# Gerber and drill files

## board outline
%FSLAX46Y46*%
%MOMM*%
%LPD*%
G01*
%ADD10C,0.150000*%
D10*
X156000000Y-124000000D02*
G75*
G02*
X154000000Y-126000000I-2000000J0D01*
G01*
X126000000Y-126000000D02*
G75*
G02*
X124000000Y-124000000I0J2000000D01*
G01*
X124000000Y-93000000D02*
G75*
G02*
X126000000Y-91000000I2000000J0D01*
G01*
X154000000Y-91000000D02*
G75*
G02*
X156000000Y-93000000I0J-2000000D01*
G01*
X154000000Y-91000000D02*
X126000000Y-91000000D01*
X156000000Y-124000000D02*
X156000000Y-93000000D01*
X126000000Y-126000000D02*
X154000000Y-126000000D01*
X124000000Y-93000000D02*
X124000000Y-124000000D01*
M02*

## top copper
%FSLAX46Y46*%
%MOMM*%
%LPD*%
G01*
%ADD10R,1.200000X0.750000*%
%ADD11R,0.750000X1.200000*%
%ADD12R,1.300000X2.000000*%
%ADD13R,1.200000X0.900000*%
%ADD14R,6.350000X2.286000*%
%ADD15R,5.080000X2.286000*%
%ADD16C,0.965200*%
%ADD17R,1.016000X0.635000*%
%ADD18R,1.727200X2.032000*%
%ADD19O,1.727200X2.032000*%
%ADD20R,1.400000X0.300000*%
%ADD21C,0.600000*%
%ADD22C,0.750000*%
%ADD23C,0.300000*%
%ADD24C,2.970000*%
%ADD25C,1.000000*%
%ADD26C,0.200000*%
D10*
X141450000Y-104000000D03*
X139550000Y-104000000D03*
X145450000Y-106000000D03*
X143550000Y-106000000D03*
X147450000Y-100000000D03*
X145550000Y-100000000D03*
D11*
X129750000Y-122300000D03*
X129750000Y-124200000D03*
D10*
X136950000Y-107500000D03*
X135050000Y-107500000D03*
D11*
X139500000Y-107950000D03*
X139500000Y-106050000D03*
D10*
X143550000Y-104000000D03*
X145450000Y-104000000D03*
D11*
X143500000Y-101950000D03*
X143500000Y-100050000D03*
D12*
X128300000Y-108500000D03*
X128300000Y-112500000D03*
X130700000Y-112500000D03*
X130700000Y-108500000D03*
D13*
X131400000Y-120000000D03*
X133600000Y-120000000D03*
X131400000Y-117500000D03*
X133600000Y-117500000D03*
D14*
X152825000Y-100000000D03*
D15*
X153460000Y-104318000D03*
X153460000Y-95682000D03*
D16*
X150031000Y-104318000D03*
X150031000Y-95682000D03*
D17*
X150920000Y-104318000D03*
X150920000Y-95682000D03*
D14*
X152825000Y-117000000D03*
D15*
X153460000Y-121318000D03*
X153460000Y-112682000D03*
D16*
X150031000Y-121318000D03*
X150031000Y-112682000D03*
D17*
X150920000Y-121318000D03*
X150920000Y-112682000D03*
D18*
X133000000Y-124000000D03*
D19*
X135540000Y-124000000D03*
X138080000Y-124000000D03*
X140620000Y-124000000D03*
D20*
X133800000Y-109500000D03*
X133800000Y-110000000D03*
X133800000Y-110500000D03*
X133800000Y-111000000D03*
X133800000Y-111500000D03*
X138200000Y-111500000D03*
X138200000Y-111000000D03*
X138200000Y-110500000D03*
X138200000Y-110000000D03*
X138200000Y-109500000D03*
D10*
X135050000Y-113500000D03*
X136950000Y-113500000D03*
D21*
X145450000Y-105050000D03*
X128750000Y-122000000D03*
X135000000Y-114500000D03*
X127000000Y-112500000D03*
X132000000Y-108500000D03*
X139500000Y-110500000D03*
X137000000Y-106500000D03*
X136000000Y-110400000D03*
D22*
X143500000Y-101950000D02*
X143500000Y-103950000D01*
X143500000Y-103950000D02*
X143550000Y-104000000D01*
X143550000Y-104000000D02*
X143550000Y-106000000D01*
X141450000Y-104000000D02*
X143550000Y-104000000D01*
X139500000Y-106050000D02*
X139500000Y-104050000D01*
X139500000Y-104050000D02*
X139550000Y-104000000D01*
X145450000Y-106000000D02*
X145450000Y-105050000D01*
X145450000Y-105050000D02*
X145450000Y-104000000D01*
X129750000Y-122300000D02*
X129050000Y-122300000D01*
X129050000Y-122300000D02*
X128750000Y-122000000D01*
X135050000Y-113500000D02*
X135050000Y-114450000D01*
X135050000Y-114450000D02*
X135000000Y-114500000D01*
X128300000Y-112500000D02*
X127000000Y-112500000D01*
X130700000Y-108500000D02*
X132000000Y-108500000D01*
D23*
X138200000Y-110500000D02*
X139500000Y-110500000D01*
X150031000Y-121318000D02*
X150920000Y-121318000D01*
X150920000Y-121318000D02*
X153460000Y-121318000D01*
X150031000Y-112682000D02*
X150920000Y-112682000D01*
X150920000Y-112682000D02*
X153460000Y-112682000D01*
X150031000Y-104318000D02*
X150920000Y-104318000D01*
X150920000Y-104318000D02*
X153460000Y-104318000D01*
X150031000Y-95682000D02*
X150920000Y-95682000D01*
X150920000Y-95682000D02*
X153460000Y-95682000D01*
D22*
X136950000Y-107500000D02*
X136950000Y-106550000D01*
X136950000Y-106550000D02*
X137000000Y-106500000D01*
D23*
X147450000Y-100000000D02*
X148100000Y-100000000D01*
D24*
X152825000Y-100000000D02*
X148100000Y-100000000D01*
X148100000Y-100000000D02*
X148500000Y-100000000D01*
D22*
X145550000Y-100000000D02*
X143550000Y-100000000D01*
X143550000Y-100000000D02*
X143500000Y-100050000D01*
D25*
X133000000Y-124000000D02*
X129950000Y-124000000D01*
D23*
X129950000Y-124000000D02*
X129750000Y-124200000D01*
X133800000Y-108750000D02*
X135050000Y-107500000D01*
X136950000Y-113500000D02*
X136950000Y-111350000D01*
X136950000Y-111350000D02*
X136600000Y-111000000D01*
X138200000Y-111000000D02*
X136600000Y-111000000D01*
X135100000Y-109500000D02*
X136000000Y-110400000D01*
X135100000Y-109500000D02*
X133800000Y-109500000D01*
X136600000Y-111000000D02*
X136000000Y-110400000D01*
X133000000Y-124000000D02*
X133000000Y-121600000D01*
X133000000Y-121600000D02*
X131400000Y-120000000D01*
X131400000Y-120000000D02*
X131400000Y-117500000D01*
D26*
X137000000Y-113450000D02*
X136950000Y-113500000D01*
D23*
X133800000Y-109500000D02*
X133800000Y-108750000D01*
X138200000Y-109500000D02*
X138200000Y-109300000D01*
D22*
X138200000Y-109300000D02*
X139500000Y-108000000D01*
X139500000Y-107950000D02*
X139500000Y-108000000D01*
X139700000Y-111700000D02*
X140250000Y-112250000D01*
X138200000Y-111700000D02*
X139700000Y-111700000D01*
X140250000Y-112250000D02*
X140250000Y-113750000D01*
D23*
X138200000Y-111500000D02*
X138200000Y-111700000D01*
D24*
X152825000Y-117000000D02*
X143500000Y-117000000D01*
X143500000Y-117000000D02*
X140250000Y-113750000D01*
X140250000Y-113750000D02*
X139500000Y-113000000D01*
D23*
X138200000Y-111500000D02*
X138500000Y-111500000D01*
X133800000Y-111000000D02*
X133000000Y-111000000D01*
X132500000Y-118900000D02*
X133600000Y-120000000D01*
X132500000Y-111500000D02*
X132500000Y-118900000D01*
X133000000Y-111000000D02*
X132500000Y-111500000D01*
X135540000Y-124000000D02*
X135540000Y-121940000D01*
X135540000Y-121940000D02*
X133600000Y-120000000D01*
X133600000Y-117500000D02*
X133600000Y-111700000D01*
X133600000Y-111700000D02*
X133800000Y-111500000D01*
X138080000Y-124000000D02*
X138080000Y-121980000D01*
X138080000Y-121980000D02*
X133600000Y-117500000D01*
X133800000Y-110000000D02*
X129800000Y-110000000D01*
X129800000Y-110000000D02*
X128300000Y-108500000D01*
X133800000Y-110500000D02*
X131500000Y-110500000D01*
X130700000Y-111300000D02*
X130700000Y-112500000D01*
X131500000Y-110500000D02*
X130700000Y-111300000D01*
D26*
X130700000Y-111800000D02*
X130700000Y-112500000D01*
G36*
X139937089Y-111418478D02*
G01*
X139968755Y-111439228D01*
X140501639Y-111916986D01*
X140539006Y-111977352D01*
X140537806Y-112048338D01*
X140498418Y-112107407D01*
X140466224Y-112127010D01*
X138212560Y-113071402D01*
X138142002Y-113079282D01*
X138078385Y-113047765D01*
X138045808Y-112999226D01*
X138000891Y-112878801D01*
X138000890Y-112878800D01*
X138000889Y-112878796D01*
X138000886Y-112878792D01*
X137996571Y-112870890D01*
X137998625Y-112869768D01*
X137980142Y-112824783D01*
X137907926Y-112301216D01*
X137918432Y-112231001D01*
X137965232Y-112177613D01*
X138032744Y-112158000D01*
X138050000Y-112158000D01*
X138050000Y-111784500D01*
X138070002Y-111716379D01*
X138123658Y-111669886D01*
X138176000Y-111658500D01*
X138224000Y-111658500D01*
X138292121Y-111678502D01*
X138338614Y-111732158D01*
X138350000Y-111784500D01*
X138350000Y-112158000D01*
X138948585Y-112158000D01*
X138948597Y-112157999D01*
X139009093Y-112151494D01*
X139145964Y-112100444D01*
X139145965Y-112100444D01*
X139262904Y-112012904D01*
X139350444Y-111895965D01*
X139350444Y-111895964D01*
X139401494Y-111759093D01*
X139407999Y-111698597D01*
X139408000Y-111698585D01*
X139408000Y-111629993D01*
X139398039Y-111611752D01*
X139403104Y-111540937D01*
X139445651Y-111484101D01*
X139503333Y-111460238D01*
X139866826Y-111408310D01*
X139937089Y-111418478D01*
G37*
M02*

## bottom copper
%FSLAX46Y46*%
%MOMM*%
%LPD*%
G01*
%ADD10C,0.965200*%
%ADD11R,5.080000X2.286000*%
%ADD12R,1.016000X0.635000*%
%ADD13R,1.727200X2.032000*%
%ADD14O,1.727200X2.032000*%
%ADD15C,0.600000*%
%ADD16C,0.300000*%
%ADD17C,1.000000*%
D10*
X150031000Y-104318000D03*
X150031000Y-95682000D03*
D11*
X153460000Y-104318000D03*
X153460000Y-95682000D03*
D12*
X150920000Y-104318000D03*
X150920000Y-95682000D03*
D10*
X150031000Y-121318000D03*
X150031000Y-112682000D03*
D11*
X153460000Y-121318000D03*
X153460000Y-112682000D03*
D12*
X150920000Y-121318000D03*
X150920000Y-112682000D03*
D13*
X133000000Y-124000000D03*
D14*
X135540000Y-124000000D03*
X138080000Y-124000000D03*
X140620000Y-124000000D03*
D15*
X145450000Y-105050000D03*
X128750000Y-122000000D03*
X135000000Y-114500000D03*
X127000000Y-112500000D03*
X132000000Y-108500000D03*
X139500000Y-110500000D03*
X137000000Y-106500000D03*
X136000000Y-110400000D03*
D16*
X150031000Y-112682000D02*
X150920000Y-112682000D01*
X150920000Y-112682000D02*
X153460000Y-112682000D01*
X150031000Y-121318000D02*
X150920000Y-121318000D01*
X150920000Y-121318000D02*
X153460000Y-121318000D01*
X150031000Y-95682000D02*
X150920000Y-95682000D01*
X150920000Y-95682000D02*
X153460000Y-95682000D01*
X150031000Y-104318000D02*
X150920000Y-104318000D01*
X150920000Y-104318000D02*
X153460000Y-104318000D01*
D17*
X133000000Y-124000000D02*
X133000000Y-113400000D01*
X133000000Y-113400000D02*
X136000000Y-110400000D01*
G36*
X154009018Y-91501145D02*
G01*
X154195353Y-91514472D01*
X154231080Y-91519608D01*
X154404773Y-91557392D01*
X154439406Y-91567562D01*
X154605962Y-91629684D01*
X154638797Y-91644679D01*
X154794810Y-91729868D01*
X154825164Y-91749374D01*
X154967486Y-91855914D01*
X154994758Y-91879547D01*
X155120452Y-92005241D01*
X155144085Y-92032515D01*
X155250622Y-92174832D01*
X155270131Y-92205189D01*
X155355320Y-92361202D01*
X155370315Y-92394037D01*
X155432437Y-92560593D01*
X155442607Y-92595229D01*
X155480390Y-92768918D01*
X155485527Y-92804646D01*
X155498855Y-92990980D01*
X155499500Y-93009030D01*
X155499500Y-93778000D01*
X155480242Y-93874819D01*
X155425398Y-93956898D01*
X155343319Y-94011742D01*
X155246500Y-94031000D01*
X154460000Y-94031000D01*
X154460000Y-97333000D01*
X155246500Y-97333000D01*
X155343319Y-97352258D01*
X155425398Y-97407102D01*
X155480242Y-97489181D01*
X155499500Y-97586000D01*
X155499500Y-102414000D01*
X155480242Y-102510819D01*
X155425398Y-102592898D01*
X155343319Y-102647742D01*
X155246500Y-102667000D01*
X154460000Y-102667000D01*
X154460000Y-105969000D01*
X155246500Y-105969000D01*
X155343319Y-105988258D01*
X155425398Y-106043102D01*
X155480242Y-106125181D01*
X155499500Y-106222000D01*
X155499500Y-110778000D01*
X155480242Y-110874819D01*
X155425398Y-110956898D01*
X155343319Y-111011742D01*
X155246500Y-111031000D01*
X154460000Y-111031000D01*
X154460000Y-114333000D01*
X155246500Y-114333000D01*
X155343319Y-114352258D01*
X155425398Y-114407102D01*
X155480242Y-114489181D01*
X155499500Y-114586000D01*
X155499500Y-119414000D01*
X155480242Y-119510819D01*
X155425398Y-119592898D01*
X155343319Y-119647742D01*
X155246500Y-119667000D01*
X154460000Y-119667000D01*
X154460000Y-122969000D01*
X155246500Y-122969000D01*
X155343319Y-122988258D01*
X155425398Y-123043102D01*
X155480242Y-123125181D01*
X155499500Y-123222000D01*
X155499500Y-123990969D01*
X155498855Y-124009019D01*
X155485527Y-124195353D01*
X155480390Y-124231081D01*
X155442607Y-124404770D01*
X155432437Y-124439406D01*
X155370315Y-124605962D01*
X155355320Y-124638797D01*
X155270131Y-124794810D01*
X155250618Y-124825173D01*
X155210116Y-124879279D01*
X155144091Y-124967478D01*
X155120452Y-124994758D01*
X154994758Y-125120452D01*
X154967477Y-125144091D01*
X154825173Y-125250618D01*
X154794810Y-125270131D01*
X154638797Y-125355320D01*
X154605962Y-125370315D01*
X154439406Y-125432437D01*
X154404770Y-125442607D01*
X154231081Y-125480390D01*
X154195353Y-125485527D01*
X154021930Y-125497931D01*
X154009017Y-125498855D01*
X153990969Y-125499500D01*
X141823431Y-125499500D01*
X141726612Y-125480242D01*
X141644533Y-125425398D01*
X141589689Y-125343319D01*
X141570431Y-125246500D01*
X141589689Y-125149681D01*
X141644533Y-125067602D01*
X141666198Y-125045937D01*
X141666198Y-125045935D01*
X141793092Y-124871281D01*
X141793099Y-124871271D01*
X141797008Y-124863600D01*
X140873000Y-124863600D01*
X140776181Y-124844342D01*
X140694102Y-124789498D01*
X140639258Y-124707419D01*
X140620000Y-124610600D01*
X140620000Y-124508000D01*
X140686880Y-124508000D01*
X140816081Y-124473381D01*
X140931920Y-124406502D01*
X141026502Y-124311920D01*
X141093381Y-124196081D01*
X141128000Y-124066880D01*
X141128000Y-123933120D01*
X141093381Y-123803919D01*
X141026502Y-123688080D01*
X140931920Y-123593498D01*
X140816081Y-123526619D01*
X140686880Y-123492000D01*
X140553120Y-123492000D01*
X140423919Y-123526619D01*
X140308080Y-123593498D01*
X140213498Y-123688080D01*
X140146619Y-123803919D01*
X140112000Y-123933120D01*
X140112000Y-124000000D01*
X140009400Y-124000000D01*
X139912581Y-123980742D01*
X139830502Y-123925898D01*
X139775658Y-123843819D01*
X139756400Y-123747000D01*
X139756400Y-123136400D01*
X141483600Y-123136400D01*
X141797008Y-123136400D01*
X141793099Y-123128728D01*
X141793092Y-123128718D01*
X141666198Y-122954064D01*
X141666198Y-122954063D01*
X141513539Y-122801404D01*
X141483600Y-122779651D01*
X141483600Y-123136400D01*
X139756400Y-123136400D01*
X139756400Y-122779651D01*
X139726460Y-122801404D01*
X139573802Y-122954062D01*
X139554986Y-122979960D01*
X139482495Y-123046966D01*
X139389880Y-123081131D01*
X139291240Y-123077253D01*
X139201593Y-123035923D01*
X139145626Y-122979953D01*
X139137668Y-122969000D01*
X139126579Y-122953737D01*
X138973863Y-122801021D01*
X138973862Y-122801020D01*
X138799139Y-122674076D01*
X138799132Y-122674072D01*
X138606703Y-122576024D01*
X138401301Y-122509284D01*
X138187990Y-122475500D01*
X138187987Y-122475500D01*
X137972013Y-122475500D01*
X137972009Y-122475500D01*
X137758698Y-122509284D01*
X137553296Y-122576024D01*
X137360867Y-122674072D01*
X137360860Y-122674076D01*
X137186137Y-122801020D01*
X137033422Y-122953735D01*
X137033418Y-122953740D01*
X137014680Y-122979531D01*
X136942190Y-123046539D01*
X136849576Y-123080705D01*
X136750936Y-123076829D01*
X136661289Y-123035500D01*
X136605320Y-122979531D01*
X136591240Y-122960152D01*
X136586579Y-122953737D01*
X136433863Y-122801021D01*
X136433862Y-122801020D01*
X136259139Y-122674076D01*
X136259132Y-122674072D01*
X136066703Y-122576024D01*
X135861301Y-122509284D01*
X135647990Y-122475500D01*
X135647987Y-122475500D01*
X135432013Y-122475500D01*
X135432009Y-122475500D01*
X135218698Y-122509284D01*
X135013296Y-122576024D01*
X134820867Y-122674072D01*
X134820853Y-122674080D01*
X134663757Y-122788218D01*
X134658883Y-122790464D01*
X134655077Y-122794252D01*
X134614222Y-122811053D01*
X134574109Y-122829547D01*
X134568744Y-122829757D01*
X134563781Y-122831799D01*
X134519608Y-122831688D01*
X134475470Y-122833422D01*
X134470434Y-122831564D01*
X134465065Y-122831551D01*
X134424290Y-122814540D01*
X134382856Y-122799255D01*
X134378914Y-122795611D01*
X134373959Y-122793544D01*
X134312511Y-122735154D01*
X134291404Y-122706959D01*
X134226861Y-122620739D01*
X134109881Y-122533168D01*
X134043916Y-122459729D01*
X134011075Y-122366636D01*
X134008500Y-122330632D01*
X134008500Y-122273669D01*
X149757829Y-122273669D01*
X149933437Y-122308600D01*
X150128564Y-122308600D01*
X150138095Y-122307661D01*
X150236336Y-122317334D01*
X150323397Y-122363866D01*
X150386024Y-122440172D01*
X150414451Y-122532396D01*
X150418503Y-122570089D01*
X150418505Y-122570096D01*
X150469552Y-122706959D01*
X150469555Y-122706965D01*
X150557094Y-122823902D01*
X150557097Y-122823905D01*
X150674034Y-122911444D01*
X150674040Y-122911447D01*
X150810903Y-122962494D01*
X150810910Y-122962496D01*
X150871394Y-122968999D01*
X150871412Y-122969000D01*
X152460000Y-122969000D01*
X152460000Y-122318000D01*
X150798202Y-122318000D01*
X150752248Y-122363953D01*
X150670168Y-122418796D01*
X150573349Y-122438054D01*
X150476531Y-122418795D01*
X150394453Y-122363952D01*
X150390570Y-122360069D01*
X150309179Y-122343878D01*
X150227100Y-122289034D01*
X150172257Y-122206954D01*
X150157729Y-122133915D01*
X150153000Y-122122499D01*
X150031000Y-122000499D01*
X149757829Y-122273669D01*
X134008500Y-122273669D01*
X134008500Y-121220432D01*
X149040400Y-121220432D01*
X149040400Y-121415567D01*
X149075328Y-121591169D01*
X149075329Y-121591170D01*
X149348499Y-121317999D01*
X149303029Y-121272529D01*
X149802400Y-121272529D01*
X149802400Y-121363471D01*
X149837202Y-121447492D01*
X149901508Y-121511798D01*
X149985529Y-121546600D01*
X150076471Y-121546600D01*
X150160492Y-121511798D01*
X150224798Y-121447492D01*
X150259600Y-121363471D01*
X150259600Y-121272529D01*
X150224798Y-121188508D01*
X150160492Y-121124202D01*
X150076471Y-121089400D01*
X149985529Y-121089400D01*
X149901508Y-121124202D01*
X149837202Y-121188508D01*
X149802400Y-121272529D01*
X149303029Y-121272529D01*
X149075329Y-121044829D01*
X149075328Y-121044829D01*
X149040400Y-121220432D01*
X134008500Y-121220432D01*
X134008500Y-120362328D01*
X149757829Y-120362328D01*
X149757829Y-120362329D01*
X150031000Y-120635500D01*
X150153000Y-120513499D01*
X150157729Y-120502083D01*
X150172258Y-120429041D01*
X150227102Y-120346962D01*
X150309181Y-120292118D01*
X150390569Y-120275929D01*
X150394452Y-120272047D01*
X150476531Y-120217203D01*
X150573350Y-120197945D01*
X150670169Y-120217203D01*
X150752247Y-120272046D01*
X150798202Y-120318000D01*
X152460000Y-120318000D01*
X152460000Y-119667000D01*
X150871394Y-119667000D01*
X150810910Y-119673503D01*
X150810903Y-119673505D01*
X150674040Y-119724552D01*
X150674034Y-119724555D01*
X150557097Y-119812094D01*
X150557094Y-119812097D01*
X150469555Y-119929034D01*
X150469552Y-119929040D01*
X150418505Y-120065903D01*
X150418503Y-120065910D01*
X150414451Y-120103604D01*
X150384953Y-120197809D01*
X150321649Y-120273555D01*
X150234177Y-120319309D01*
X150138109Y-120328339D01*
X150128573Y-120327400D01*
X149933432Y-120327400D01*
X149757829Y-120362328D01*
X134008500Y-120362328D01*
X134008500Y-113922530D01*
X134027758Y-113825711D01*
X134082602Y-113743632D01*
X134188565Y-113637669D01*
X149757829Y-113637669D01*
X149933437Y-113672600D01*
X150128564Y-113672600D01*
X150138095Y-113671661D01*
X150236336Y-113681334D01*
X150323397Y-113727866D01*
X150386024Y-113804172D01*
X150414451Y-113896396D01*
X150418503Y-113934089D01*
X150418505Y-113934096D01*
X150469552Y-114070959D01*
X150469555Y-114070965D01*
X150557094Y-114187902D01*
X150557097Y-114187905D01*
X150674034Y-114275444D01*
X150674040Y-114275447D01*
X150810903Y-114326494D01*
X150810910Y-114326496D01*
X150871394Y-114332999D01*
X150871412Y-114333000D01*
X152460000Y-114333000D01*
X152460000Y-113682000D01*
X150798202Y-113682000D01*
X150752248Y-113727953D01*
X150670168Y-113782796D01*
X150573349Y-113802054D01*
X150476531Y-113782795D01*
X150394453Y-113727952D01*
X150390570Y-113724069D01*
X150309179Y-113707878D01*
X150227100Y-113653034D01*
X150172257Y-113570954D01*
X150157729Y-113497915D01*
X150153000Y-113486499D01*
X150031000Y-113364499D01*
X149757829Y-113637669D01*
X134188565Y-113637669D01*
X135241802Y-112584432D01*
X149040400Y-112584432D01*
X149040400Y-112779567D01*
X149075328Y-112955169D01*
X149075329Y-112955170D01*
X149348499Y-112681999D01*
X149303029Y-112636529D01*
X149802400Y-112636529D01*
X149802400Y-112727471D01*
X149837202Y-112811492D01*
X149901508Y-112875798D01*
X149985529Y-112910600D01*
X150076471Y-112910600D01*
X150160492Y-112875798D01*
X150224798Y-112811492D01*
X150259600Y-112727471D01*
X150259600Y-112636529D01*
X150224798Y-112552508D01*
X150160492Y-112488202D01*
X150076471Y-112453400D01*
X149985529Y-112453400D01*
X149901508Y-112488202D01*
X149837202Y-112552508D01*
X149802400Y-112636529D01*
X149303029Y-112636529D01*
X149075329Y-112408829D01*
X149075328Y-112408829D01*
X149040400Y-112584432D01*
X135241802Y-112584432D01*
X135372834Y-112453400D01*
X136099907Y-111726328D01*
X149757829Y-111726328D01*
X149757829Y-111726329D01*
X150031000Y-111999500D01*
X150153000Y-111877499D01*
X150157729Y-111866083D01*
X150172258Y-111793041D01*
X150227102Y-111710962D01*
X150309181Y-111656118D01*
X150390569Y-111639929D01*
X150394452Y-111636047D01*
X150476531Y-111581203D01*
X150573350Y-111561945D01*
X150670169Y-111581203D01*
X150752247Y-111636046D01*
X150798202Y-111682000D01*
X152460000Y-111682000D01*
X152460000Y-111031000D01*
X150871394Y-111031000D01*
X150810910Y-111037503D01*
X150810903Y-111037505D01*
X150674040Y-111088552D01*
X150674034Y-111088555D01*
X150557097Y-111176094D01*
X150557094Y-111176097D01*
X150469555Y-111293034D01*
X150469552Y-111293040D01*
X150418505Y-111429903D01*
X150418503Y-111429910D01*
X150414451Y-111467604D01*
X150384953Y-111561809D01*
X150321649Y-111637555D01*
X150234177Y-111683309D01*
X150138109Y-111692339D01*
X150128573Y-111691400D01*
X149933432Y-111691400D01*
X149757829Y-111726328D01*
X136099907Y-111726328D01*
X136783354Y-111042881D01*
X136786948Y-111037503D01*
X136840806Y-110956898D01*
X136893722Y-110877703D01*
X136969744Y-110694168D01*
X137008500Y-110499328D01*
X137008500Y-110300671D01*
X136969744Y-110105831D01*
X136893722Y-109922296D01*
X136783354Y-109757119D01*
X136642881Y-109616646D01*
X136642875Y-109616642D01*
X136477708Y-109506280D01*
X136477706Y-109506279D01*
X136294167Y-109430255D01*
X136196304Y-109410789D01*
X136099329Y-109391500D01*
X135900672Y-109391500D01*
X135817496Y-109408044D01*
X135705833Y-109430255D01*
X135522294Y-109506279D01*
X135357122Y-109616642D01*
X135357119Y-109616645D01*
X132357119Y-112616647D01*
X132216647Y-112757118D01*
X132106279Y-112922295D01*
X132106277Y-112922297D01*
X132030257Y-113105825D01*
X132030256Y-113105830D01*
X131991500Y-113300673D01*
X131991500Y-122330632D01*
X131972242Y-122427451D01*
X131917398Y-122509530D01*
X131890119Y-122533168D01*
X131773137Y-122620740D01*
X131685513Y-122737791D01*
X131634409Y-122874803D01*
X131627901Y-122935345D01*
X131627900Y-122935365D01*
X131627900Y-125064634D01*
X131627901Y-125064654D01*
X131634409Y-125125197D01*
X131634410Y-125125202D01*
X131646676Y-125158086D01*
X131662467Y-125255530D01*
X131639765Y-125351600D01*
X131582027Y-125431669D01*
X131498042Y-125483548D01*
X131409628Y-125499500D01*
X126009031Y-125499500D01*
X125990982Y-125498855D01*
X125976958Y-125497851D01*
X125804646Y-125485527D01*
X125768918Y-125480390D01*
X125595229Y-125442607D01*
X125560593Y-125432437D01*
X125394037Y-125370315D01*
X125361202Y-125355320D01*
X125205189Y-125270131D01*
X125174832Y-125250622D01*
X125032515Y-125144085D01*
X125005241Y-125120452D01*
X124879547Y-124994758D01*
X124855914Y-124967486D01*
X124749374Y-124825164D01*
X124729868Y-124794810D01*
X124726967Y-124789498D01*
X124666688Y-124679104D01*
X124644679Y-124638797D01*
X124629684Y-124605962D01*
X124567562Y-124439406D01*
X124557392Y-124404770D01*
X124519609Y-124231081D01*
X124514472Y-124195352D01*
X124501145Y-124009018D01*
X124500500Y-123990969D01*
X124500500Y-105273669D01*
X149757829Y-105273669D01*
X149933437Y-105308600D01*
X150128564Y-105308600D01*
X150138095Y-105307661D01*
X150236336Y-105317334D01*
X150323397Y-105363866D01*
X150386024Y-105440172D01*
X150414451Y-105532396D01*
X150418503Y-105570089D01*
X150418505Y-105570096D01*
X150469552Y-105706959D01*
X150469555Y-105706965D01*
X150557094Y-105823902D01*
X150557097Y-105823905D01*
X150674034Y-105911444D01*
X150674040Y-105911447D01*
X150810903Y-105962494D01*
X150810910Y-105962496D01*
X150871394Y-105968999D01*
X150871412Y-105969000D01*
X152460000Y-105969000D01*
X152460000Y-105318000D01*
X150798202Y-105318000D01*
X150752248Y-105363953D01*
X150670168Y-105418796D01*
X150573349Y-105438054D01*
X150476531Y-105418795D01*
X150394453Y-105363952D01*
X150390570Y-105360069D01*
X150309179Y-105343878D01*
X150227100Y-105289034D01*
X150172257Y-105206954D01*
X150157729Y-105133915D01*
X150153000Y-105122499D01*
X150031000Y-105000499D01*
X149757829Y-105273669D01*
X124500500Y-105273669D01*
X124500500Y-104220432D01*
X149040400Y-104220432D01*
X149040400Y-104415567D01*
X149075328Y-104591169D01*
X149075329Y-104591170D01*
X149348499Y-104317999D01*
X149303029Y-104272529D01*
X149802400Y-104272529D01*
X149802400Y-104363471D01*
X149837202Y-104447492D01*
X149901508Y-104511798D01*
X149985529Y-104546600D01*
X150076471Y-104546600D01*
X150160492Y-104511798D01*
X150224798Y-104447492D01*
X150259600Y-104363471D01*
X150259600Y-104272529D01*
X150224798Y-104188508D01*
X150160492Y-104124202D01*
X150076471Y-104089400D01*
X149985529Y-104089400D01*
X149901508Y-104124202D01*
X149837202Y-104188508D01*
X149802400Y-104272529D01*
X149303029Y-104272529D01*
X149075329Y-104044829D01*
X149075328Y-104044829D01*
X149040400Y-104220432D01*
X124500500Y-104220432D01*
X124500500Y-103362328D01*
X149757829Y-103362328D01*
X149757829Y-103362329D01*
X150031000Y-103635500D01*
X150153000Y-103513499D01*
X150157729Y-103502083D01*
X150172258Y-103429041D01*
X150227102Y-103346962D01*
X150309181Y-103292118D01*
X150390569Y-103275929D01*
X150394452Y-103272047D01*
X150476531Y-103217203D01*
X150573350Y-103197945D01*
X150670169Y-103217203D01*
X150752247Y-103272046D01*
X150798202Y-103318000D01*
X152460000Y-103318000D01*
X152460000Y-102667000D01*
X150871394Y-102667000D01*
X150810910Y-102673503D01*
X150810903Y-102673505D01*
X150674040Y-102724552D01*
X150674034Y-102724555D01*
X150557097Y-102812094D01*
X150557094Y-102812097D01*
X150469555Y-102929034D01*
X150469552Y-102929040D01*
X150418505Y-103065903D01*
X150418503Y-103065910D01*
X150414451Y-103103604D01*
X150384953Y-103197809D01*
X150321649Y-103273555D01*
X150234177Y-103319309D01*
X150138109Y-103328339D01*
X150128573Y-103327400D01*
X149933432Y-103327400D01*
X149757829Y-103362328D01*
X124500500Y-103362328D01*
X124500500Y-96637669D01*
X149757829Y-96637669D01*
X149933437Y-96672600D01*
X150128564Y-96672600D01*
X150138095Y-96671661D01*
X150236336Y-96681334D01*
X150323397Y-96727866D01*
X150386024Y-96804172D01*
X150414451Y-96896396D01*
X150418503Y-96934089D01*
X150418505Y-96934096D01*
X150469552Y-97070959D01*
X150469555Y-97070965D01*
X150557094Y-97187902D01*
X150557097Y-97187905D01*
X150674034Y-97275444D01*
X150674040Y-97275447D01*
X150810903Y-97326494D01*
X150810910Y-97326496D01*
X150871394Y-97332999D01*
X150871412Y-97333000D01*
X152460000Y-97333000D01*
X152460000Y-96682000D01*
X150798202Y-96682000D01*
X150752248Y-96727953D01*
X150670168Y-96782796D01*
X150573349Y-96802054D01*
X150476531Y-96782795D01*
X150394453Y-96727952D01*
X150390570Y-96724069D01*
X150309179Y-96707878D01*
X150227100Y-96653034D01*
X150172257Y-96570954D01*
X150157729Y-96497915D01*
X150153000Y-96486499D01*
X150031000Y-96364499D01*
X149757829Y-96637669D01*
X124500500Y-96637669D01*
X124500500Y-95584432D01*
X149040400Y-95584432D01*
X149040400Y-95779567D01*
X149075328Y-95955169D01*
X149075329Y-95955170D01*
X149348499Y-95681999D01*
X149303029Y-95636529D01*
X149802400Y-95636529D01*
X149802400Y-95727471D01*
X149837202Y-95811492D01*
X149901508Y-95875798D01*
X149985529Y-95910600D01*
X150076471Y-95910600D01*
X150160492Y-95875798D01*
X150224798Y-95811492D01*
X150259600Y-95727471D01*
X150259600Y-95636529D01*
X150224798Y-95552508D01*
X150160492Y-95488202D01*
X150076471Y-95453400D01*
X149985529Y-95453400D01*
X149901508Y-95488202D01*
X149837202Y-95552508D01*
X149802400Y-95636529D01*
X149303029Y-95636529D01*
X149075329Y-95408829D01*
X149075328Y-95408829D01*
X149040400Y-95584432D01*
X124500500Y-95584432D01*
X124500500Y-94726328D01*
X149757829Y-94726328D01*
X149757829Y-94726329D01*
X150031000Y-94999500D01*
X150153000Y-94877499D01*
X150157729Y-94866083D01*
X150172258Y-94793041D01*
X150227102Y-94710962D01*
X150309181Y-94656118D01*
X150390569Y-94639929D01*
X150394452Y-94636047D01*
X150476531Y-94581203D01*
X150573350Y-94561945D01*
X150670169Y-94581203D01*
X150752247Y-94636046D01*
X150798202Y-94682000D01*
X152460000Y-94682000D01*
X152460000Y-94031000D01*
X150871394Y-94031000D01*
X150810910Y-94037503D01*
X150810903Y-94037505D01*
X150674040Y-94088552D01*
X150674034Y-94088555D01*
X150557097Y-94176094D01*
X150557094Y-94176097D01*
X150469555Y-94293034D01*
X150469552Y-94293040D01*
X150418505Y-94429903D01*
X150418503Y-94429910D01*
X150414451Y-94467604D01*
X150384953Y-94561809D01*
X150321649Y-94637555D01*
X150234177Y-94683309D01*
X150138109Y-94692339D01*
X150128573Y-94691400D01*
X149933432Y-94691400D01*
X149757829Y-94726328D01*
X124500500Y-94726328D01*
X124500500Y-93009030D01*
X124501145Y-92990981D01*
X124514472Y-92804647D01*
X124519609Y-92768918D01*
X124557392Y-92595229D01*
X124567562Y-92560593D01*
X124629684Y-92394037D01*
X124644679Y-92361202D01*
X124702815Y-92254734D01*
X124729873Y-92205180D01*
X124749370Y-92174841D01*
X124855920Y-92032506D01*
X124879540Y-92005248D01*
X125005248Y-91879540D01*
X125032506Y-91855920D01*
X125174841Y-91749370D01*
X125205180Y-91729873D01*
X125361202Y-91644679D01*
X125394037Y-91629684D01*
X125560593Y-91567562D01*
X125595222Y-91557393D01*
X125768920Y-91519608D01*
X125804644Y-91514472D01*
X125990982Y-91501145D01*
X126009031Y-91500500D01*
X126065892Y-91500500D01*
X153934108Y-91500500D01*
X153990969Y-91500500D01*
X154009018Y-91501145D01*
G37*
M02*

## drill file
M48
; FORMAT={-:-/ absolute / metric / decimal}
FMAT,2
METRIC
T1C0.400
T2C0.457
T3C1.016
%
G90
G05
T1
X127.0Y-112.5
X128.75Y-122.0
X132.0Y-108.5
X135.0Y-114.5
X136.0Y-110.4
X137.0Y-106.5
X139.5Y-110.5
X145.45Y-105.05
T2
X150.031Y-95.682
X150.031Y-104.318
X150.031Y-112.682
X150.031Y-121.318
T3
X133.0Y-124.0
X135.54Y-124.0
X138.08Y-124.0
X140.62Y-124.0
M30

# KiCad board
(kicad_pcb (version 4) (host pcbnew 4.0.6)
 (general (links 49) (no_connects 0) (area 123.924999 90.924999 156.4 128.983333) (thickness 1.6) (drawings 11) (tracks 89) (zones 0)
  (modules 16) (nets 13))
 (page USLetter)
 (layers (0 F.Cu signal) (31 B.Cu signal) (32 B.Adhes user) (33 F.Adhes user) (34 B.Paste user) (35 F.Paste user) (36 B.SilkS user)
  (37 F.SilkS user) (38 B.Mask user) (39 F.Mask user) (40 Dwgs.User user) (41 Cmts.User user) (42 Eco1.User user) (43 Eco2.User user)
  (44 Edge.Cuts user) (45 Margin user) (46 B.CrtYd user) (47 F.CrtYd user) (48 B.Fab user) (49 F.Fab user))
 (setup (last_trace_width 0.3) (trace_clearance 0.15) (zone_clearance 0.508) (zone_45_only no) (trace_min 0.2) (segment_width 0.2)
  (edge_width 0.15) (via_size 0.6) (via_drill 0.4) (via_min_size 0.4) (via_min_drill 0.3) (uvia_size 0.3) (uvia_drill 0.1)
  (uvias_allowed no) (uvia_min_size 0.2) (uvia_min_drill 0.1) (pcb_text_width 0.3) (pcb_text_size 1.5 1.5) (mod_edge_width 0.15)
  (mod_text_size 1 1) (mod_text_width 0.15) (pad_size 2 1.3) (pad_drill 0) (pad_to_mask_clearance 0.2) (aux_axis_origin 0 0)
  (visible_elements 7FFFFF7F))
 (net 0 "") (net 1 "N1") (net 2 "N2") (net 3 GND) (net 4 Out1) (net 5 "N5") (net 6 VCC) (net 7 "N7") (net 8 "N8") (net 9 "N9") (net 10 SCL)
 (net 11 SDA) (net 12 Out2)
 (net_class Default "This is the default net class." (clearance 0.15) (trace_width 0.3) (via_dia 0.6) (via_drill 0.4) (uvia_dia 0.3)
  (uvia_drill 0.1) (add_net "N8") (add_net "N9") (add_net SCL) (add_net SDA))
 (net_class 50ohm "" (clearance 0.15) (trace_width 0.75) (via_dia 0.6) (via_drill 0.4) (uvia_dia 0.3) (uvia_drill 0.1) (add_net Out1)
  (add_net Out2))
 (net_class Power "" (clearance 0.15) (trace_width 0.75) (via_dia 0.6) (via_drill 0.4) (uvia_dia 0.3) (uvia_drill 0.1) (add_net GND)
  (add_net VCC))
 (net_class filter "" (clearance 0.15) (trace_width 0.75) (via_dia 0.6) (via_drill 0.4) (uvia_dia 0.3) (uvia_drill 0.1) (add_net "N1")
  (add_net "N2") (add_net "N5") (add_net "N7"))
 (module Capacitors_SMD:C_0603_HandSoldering (layer F.Cu) (at 140.5 104 180)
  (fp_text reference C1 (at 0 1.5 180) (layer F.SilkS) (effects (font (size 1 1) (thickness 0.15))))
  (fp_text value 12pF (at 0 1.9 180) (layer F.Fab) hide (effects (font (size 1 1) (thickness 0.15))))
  (pad 1 smd rect (at -0.95 0 180) (size 1.2 0.75) (layers F.Cu F.Paste F.Mask) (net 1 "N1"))
  (pad 2 smd rect (at 0.95 0 180) (size 1.2 0.75) (layers F.Cu F.Paste F.Mask) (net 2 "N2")))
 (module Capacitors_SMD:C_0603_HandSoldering (layer F.Cu) (at 144.5 106 180)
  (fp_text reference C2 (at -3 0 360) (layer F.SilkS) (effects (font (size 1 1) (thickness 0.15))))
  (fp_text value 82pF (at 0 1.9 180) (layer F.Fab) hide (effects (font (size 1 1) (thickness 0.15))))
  (pad 1 smd rect (at -0.95 0 180) (size 1.2 0.75) (layers F.Cu F.Paste F.Mask) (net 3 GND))
  (pad 2 smd rect (at 0.95 0 180) (size 1.2 0.75) (layers F.Cu F.Paste F.Mask) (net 1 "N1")))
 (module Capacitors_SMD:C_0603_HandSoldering (layer F.Cu) (at 146.5 100 180)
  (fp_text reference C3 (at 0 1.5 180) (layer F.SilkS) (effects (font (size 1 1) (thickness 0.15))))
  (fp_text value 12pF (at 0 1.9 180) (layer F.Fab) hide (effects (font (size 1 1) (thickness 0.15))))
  (pad 1 smd rect (at -0.95 0 180) (size 1.2 0.75) (layers F.Cu F.Paste F.Mask) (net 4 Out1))
  (pad 2 smd rect (at 0.95 0 180) (size 1.2 0.75) (layers F.Cu F.Paste F.Mask) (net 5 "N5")))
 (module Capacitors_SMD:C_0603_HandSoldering (layer F.Cu) (at 129.75 123.25 270)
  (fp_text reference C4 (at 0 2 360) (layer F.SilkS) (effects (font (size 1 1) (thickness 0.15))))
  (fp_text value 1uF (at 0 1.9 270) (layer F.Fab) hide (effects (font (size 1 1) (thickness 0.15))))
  (pad 1 smd rect (at -0.95 0 270) (size 1.2 0.75) (layers F.Cu F.Paste F.Mask) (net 3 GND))
  (pad 2 smd rect (at 0.95 0 270) (size 1.2 0.75) (layers F.Cu F.Paste F.Mask) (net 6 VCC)))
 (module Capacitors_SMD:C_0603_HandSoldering (layer F.Cu) (at 136 107.5 180)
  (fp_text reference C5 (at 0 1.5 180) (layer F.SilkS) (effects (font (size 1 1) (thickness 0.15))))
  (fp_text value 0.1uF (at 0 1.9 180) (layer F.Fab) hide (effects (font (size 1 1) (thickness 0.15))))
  (pad 1 smd rect (at -0.95 0 180) (size 1.2 0.75) (layers F.Cu F.Paste F.Mask) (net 3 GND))
  (pad 2 smd rect (at 0.95 0 180) (size 1.2 0.75) (layers F.Cu F.Paste F.Mask) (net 6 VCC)))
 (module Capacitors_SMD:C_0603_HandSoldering (layer F.Cu) (at 139.5 107 90)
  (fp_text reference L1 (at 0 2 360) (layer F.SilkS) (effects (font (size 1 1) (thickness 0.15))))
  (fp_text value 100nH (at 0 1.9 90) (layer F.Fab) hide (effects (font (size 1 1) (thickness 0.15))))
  (pad 1 smd rect (at -0.95 0 90) (size 1.2 0.75) (layers F.Cu F.Paste F.Mask) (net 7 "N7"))
  (pad 2 smd rect (at 0.95 0 90) (size 1.2 0.75) (layers F.Cu F.Paste F.Mask) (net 2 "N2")))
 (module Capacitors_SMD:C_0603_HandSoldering (layer F.Cu) (at 144.5 104)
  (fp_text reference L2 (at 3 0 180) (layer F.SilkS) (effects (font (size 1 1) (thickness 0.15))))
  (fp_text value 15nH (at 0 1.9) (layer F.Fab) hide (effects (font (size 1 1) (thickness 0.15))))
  (pad 1 smd rect (at -0.95 0) (size 1.2 0.75) (layers F.Cu F.Paste F.Mask) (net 1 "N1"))
  (pad 2 smd rect (at 0.95 0) (size 1.2 0.75) (layers F.Cu F.Paste F.Mask) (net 3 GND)))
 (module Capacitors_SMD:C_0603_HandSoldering (layer F.Cu) (at 143.5 101 90)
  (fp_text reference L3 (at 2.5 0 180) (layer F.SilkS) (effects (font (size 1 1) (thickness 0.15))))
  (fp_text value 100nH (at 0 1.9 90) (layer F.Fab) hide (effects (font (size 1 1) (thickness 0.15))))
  (pad 1 smd rect (at -0.95 0 90) (size 1.2 0.75) (layers F.Cu F.Paste F.Mask) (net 1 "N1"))
  (pad 2 smd rect (at 0.95 0 90) (size 1.2 0.75) (layers F.Cu F.Paste F.Mask) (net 5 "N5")))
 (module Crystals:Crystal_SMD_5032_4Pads (layer F.Cu) (at 129.5 110.5 270)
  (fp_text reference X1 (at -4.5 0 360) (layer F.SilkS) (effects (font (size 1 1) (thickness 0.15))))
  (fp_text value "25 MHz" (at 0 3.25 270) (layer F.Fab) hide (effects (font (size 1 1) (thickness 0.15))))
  (pad 1 smd rect (at -2 1.2 270) (size 2 1.3) (layers F.Cu F.Paste F.Mask) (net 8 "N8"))
  (pad 3 smd rect (at 2 1.2 270) (size 2 1.3) (layers F.Cu F.Paste F.Mask) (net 3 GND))
  (pad 2 smd rect (at 2 -1.2 270) (size 2 1.3) (layers F.Cu F.Paste F.Mask) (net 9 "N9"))
  (pad 3 smd rect (at -2 -1.2 270) (size 2 1.3) (layers F.Cu F.Paste F.Mask) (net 3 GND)))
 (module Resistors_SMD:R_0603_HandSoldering (layer F.Cu) (at 132.5 120)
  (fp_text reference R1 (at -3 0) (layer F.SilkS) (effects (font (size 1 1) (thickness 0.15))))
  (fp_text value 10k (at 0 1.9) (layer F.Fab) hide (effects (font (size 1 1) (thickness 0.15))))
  (pad 1 smd rect (at -1.1 0) (size 1.2 0.9) (layers F.Cu F.Paste F.Mask) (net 6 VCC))
  (pad 2 smd rect (at 1.1 0) (size 1.2 0.9) (layers F.Cu F.Paste F.Mask) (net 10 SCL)))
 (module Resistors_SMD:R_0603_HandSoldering (layer F.Cu) (at 132.5 117.5)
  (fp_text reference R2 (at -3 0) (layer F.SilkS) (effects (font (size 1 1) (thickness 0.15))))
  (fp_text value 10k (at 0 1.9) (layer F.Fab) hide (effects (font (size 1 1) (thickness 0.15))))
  (pad 1 smd rect (at -1.1 0) (size 1.2 0.9) (layers F.Cu F.Paste F.Mask) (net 6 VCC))
  (pad 2 smd rect (at 1.1 0) (size 1.2 0.9) (layers F.Cu F.Paste F.Mask) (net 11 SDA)))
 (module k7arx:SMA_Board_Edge (layer F.Cu) (at 156 100 180)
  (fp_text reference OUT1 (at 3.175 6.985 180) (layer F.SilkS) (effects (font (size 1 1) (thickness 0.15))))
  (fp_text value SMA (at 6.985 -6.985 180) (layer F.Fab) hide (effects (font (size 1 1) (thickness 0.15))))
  (pad 1 smd rect (at 3.175 0 180) (size 6.35 2.286) (layers F.Cu F.Paste F.Mask) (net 4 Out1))
  (pad 2 smd rect (at 2.54 -4.318 180) (size 5.08 2.286) (layers F.Cu F.Paste F.Mask) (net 3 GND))
  (pad 2 smd rect (at 2.54 4.318 180) (size 5.08 2.286) (layers F.Cu F.Paste F.Mask) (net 3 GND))
  (pad 2 thru_hole circle (at 5.969 -4.318 180) (size 0.9652 0.9652) (drill 0.4572) (layers *.Cu *.Mask F.SilkS) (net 3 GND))
  (pad 2 thru_hole circle (at 5.969 4.318 180) (size 0.9652 0.9652) (drill 0.4572) (layers *.Cu *.Mask F.SilkS) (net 3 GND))
  (pad 2 smd rect (at 5.08 -4.318 180) (size 1.016 0.635) (layers F.Cu F.Paste F.Mask) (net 3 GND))
  (pad 2 smd rect (at 5.08 4.318 180) (size 1.016 0.635) (layers F.Cu F.Paste F.Mask) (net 3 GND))
  (pad 2 smd rect (at 2.54 -4.318 180) (size 5.08 2.286) (layers B.Cu B.Paste B.Mask) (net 3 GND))
  (pad 2 smd rect (at 2.54 4.318 180) (size 5.08 2.286) (layers B.Cu B.Paste B.Mask) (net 3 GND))
  (pad 2 smd rect (at 5.08 -4.318 180) (size 1.016 0.635) (layers B.Cu B.Paste B.Mask) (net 3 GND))
  (pad 2 smd rect (at 5.08 4.318 180) (size 1.016 0.635) (layers B.Cu B.Paste B.Mask) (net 3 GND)))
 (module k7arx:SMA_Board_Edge (layer F.Cu) (at 156 117 180)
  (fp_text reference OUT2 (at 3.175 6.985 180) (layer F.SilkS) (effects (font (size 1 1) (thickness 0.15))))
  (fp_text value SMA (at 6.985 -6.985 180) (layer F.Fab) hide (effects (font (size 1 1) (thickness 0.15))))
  (pad 1 smd rect (at 3.175 0 180) (size 6.35 2.286) (layers F.Cu F.Paste F.Mask) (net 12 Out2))
  (pad 2 smd rect (at 2.54 -4.318 180) (size 5.08 2.286) (layers F.Cu F.Paste F.Mask) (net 3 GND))
  (pad 2 smd rect (at 2.54 4.318 180) (size 5.08 2.286) (layers F.Cu F.Paste F.Mask) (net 3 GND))
  (pad 2 thru_hole circle (at 5.969 -4.318 180) (size 0.9652 0.9652) (drill 0.4572) (layers *.Cu *.Mask F.SilkS) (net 3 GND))
  (pad 2 thru_hole circle (at 5.969 4.318 180) (size 0.9652 0.9652) (drill 0.4572) (layers *.Cu *.Mask F.SilkS) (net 3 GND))
  (pad 2 smd rect (at 5.08 -4.318 180) (size 1.016 0.635) (layers F.Cu F.Paste F.Mask) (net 3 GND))
  (pad 2 smd rect (at 5.08 4.318 180) (size 1.016 0.635) (layers F.Cu F.Paste F.Mask) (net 3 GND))
  (pad 2 smd rect (at 2.54 -4.318 180) (size 5.08 2.286) (layers B.Cu B.Paste B.Mask) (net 3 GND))
  (pad 2 smd rect (at 2.54 4.318 180) (size 5.08 2.286) (layers B.Cu B.Paste B.Mask) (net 3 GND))
  (pad 2 smd rect (at 5.08 -4.318 180) (size 1.016 0.635) (layers B.Cu B.Paste B.Mask) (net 3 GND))
  (pad 2 smd rect (at 5.08 4.318 180) (size 1.016 0.635) (layers B.Cu B.Paste B.Mask) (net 3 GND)))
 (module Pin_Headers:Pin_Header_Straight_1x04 (layer F.Cu) (at 133 124 90)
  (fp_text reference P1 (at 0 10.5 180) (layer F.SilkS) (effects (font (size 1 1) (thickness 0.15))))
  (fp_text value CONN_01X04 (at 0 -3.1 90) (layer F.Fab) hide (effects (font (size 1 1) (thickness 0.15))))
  (pad 1 thru_hole rect (at 0 0 90) (size 2.032 1.7272) (drill 1.016) (layers *.Cu *.Mask) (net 6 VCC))
  (pad 2 thru_hole oval (at 0 2.54 90) (size 2.032 1.7272) (drill 1.016) (layers *.Cu *.Mask) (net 10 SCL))
  (pad 3 thru_hole oval (at 0 5.08 90) (size 2.032 1.7272) (drill 1.016) (layers *.Cu *.Mask) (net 11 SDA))
  (pad 4 thru_hole oval (at 0 7.62 90) (size 2.032 1.7272) (drill 1.016) (layers *.Cu *.Mask) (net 3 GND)))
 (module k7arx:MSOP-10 (layer F.Cu) (at 136 110.5)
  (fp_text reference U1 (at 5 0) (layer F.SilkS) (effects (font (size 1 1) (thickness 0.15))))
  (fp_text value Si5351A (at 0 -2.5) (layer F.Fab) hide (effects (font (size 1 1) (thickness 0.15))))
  (pad 1 smd rect (at -2.2 -1) (size 1.4 0.3) (layers F.Cu F.Paste F.Mask) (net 6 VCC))
  (pad 2 smd rect (at -2.2 -0.5) (size 1.4 0.3) (layers F.Cu F.Paste F.Mask) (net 8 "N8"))
  (pad 3 smd rect (at -2.2 0) (size 1.4 0.3) (layers F.Cu F.Paste F.Mask) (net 9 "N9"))
  (pad 4 smd rect (at -2.2 0.5) (size 1.4 0.3) (layers F.Cu F.Paste F.Mask) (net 10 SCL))
  (pad 5 smd rect (at -2.2 1) (size 1.4 0.3) (layers F.Cu F.Paste F.Mask) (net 11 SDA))
  (pad 6 smd rect (at 2.2 1) (size 1.4 0.3) (layers F.Cu F.Paste F.Mask) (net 12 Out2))
  (pad 7 smd rect (at 2.2 0.5) (size 1.4 0.3) (layers F.Cu F.Paste F.Mask) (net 6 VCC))
  (pad 8 smd rect (at 2.2 0) (size 1.4 0.3) (layers F.Cu F.Paste F.Mask) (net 3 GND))
  (pad 9 smd rect (at 2.2 -0.5) (size 1.4 0.3) (layers F.Cu F.Paste F.Mask))
  (pad 10 smd rect (at 2.2 -1) (size 1.4 0.3) (layers F.Cu F.Paste F.Mask) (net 7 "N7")))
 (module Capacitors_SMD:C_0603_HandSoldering (layer F.Cu) (at 136 113.5)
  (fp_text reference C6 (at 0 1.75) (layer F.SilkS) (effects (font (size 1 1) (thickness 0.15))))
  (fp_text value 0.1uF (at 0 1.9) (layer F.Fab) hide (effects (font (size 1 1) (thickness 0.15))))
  (pad 1 smd rect (at -0.95 0) (size 1.2 0.75) (layers F.Cu F.Paste F.Mask) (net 3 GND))
  (pad 2 smd rect (at 0.95 0) (size 1.2 0.75) (layers F.Cu F.Paste F.Mask) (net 6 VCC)))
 (gr_arc (start 154 124) (end 156 124) (angle 90) (layer Edge.Cuts) (width 0.15))
 (gr_arc (start 126 124) (end 126 126) (angle 90) (layer Edge.Cuts) (width 0.15))
 (gr_arc (start 126 93) (end 124 93) (angle 90) (layer Edge.Cuts) (width 0.15))
 (gr_arc (start 154 93) (end 154 91) (angle 90) (layer Edge.Cuts) (width 0.15))
 (gr_line (start 154 91) (end 126 91) (angle 90) (layer Edge.Cuts) (width 0.15))
 (gr_line (start 156 124) (end 156 93) (angle 90) (layer Edge.Cuts) (width 0.15))
 (gr_line (start 126 126) (end 154 126) (angle 90) (layer Edge.Cuts) (width 0.15))
 (gr_line (start 124 93) (end 124 124) (angle 90) (layer Edge.Cuts) (width 0.15))
 (segment (start 143.5 101.95) (end 143.5 103.95) (width 0.75) (layer F.Cu) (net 1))
 (segment (start 143.5 103.95) (end 143.55 104) (width 0.75) (layer F.Cu) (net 1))
 (segment (start 143.55 104) (end 143.55 106) (width 0.75) (layer F.Cu) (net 1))
 (segment (start 141.45 104) (end 143.55 104) (width 0.75) (layer F.Cu) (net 1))
 (segment (start 139.5 106.05) (end 139.5 104.05) (width 0.75) (layer F.Cu) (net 2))
 (segment (start 139.5 104.05) (end 139.55 104) (width 0.75) (layer F.Cu) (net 2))
 (via (at 145.45 105.05) (size 0.6) (drill 0.4) (layers F.Cu B.Cu) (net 3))
 (segment (start 145.45 106) (end 145.45 105.05) (width 0.75) (layer F.Cu) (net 3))
 (segment (start 145.45 105.05) (end 145.45 104) (width 0.75) (layer F.Cu) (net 3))
 (segment (start 129.75 122.3) (end 129.05 122.3) (width 0.75) (layer F.Cu) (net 3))
 (via (at 128.75 122) (size 0.6) (drill 0.4) (layers F.Cu B.Cu) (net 3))
 (segment (start 129.05 122.3) (end 128.75 122) (width 0.75) (layer F.Cu) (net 3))
 (segment (start 135.05 113.5) (end 135.05 114.45) (width 0.75) (layer F.Cu) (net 3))
 (via (at 135 114.5) (size 0.6) (drill 0.4) (layers F.Cu B.Cu) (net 3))
 (segment (start 135.05 114.45) (end 135 114.5) (width 0.75) (layer F.Cu) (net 3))
 (segment (start 128.3 112.5) (end 127 112.5) (width 0.75) (layer F.Cu) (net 3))
 (via (at 127 112.5) (size 0.6) (drill 0.4) (layers F.Cu B.Cu) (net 3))
 (segment (start 130.7 108.5) (end 132 108.5) (width 0.75) (layer F.Cu) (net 3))
 (via (at 132 108.5) (size 0.6) (drill 0.4) (layers F.Cu B.Cu) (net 3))
 (segment (start 138.2 110.5) (end 139.5 110.5) (width 0.3) (layer F.Cu) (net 3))
 (via (at 139.5 110.5) (size 0.6) (drill 0.4) (layers F.Cu B.Cu) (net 3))
 (segment (start 150.031 121.318) (end 150.92 121.318) (width 0.3) (layer F.Cu) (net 3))
 (segment (start 150.92 121.318) (end 153.46 121.318) (width 0.3) (layer F.Cu) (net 3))
 (segment (start 150.031 112.682) (end 150.92 112.682) (width 0.3) (layer F.Cu) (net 3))
 (segment (start 150.92 112.682) (end 153.46 112.682) (width 0.3) (layer F.Cu) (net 3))
 (segment (start 150.031 112.682) (end 150.92 112.682) (width 0.3) (layer B.Cu) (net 3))
 (segment (start 150.92 112.682) (end 153.46 112.682) (width 0.3) (layer B.Cu) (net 3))
 (segment (start 150.031 121.318) (end 150.92 121.318) (width 0.3) (layer B.Cu) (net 3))
 (segment (start 150.92 121.318) (end 153.46 121.318) (width 0.3) (layer B.Cu) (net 3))
 (segment (start 150.031 104.318) (end 150.92 104.318) (width 0.3) (layer F.Cu) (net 3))
 (segment (start 150.92 104.318) (end 153.46 104.318) (width 0.3) (layer F.Cu) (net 3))
 (segment (start 150.031 95.682) (end 150.92 95.682) (width 0.3) (layer F.Cu) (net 3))
 (segment (start 150.92 95.682) (end 153.46 95.682) (width 0.3) (layer F.Cu) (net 3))
 (segment (start 150.031 95.682) (end 150.92 95.682) (width 0.3) (layer B.Cu) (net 3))
 (segment (start 150.92 95.682) (end 153.46 95.682) (width 0.3) (layer B.Cu) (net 3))
 (segment (start 150.031 104.318) (end 150.92 104.318) (width 0.3) (layer B.Cu) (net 3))
 (segment (start 150.92 104.318) (end 153.46 104.318) (width 0.3) (layer B.Cu) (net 3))
 (segment (start 136.95 107.5) (end 136.95 106.55) (width 0.75) (layer F.Cu) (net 3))
 (via (at 137 106.5) (size 0.6) (drill 0.4) (layers F.Cu B.Cu) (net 3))
 (segment (start 136.95 106.55) (end 137 106.5) (width 0.75) (layer F.Cu) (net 3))
 (segment (start 147.45 100) (end 148.1 100) (width 0.3) (layer F.Cu) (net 4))
 (segment (start 152.825 100) (end 148.1 100) (width 2.97) (layer F.Cu) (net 4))
 (segment (start 148.1 100) (end 148.5 100) (width 2.97) (layer F.Cu) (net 4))
 (segment (start 145.55 100) (end 143.55 100) (width 0.75) (layer F.Cu) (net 5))
 (segment (start 143.55 100) (end 143.5 100.05) (width 0.75) (layer F.Cu) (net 5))
 (segment (start 133 124) (end 129.95 124) (width 1) (layer F.Cu) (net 6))
 (segment (start 129.95 124) (end 129.75 124.2) (width 0.3) (layer F.Cu) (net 6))
 (segment (start 133.8 108.75) (end 135.05 107.5) (width 0.3) (layer F.Cu) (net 6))
 (segment (start 133 124) (end 133 113.4) (width 1) (layer B.Cu) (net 6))
 (via (at 136 110.4) (size 0.6) (drill 0.4) (layers F.Cu B.Cu) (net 6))
 (segment (start 133 113.4) (end 136 110.4) (width 1) (layer B.Cu) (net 6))
 (segment (start 136.95 113.5) (end 136.95 111.35) (width 0.3) (layer F.Cu) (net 6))
 (segment (start 136.95 111.35) (end 136.6 111) (width 0.3) (layer F.Cu) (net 6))
 (segment (start 138.2 111) (end 136.6 111) (width 0.3) (layer F.Cu) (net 6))
 (segment (start 135.1 109.5) (end 136 110.4) (width 0.3) (layer F.Cu) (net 6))
 (segment (start 135.1 109.5) (end 133.8 109.5) (width 0.3) (layer F.Cu) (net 6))
 (segment (start 136.6 111) (end 136 110.4) (width 0.3) (layer F.Cu) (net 6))
 (segment (start 133 124) (end 133 121.6) (width 0.3) (layer F.Cu) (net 6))
 (segment (start 133 121.6) (end 131.4 120) (width 0.3) (layer F.Cu) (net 6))
 (segment (start 131.4 120) (end 131.4 117.5) (width 0.3) (layer F.Cu) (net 6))
 (segment (start 137 113.45) (end 136.95 113.5) (width 0.2) (layer F.Cu) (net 6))
 (segment (start 133.8 109.5) (end 133.8 108.75) (width 0.3) (layer F.Cu) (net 6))
 (segment (start 138.2 109.5) (end 138.2 109.3) (width 0.3) (layer F.Cu) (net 7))
 (segment (start 138.2 109.3) (end 139.5 108) (width 0.75) (layer F.Cu) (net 7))
 (segment (start 139.5 107.95) (end 139.5 108) (width 0.75) (layer F.Cu) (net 7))
 (segment (start 139.7 111.7) (end 140.25 112.25) (width 0.75) (layer F.Cu) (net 12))
 (segment (start 138.2 111.7) (end 139.7 111.7) (width 0.75) (layer F.Cu) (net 12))
 (segment (start 140.25 112.25) (end 140.25 113.75) (width 0.75) (layer F.Cu) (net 12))
 (segment (start 138.2 111.5) (end 138.2 111.7) (width 0.3) (layer F.Cu) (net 12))
 (segment (start 152.825 117) (end 143.5 117) (width 2.97) (layer F.Cu) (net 12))
 (segment (start 143.5 117) (end 140.25 113.75) (width 2.97) (layer F.Cu) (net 12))
 (segment (start 140.25 113.75) (end 139.5 113) (width 2.97) (layer F.Cu) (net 12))
 (segment (start 138.2 111.5) (end 138.5 111.5) (width 0.3) (layer F.Cu) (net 12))
 (segment (start 133.8 111) (end 133 111) (width 0.3) (layer F.Cu) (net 10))
 (segment (start 132.5 118.9) (end 133.6 120) (width 0.3) (layer F.Cu) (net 10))
 (segment (start 132.5 111.5) (end 132.5 118.9) (width 0.3) (layer F.Cu) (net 10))
 (segment (start 133 111) (end 132.5 111.5) (width 0.3) (layer F.Cu) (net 10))
 (segment (start 135.54 124) (end 135.54 121.94) (width 0.3) (layer F.Cu) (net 10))
 (segment (start 135.54 121.94) (end 133.6 120) (width 0.3) (layer F.Cu) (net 10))
 (segment (start 133.6 117.5) (end 133.6 111.7) (width 0.3) (layer F.Cu) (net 11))
 (segment (start 133.6 111.7) (end 133.8 111.5) (width 0.3) (layer F.Cu) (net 11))
 (segment (start 138.08 124) (end 138.08 121.98) (width 0.3) (layer F.Cu) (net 11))
 (segment (start 138.08 121.98) (end 133.6 117.5) (width 0.3) (layer F.Cu) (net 11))
 (segment (start 133.8 110) (end 129.8 110) (width 0.3) (layer F.Cu) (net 8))
 (segment (start 129.8 110) (end 128.3 108.5) (width 0.3) (layer F.Cu) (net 8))
 (segment (start 133.8 110.5) (end 131.5 110.5) (width 0.3) (layer F.Cu) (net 9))
 (segment (start 130.7 111.3) (end 130.7 112.5) (width 0.3) (layer F.Cu) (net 9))
 (segment (start 131.5 110.5) (end 130.7 111.3) (width 0.3) (layer F.Cu) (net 9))
 (segment (start 130.7 111.8) (end 130.7 112.5) (width 0.2) (layer F.Cu) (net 9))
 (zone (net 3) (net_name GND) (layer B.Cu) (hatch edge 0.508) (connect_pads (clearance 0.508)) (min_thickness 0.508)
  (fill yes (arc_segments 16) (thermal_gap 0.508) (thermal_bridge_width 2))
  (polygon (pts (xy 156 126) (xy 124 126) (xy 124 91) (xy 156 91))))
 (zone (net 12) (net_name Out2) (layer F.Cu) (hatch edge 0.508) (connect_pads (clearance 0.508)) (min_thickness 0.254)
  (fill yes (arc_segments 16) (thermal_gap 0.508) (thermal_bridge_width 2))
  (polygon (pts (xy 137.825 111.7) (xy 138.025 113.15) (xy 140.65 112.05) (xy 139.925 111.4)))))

